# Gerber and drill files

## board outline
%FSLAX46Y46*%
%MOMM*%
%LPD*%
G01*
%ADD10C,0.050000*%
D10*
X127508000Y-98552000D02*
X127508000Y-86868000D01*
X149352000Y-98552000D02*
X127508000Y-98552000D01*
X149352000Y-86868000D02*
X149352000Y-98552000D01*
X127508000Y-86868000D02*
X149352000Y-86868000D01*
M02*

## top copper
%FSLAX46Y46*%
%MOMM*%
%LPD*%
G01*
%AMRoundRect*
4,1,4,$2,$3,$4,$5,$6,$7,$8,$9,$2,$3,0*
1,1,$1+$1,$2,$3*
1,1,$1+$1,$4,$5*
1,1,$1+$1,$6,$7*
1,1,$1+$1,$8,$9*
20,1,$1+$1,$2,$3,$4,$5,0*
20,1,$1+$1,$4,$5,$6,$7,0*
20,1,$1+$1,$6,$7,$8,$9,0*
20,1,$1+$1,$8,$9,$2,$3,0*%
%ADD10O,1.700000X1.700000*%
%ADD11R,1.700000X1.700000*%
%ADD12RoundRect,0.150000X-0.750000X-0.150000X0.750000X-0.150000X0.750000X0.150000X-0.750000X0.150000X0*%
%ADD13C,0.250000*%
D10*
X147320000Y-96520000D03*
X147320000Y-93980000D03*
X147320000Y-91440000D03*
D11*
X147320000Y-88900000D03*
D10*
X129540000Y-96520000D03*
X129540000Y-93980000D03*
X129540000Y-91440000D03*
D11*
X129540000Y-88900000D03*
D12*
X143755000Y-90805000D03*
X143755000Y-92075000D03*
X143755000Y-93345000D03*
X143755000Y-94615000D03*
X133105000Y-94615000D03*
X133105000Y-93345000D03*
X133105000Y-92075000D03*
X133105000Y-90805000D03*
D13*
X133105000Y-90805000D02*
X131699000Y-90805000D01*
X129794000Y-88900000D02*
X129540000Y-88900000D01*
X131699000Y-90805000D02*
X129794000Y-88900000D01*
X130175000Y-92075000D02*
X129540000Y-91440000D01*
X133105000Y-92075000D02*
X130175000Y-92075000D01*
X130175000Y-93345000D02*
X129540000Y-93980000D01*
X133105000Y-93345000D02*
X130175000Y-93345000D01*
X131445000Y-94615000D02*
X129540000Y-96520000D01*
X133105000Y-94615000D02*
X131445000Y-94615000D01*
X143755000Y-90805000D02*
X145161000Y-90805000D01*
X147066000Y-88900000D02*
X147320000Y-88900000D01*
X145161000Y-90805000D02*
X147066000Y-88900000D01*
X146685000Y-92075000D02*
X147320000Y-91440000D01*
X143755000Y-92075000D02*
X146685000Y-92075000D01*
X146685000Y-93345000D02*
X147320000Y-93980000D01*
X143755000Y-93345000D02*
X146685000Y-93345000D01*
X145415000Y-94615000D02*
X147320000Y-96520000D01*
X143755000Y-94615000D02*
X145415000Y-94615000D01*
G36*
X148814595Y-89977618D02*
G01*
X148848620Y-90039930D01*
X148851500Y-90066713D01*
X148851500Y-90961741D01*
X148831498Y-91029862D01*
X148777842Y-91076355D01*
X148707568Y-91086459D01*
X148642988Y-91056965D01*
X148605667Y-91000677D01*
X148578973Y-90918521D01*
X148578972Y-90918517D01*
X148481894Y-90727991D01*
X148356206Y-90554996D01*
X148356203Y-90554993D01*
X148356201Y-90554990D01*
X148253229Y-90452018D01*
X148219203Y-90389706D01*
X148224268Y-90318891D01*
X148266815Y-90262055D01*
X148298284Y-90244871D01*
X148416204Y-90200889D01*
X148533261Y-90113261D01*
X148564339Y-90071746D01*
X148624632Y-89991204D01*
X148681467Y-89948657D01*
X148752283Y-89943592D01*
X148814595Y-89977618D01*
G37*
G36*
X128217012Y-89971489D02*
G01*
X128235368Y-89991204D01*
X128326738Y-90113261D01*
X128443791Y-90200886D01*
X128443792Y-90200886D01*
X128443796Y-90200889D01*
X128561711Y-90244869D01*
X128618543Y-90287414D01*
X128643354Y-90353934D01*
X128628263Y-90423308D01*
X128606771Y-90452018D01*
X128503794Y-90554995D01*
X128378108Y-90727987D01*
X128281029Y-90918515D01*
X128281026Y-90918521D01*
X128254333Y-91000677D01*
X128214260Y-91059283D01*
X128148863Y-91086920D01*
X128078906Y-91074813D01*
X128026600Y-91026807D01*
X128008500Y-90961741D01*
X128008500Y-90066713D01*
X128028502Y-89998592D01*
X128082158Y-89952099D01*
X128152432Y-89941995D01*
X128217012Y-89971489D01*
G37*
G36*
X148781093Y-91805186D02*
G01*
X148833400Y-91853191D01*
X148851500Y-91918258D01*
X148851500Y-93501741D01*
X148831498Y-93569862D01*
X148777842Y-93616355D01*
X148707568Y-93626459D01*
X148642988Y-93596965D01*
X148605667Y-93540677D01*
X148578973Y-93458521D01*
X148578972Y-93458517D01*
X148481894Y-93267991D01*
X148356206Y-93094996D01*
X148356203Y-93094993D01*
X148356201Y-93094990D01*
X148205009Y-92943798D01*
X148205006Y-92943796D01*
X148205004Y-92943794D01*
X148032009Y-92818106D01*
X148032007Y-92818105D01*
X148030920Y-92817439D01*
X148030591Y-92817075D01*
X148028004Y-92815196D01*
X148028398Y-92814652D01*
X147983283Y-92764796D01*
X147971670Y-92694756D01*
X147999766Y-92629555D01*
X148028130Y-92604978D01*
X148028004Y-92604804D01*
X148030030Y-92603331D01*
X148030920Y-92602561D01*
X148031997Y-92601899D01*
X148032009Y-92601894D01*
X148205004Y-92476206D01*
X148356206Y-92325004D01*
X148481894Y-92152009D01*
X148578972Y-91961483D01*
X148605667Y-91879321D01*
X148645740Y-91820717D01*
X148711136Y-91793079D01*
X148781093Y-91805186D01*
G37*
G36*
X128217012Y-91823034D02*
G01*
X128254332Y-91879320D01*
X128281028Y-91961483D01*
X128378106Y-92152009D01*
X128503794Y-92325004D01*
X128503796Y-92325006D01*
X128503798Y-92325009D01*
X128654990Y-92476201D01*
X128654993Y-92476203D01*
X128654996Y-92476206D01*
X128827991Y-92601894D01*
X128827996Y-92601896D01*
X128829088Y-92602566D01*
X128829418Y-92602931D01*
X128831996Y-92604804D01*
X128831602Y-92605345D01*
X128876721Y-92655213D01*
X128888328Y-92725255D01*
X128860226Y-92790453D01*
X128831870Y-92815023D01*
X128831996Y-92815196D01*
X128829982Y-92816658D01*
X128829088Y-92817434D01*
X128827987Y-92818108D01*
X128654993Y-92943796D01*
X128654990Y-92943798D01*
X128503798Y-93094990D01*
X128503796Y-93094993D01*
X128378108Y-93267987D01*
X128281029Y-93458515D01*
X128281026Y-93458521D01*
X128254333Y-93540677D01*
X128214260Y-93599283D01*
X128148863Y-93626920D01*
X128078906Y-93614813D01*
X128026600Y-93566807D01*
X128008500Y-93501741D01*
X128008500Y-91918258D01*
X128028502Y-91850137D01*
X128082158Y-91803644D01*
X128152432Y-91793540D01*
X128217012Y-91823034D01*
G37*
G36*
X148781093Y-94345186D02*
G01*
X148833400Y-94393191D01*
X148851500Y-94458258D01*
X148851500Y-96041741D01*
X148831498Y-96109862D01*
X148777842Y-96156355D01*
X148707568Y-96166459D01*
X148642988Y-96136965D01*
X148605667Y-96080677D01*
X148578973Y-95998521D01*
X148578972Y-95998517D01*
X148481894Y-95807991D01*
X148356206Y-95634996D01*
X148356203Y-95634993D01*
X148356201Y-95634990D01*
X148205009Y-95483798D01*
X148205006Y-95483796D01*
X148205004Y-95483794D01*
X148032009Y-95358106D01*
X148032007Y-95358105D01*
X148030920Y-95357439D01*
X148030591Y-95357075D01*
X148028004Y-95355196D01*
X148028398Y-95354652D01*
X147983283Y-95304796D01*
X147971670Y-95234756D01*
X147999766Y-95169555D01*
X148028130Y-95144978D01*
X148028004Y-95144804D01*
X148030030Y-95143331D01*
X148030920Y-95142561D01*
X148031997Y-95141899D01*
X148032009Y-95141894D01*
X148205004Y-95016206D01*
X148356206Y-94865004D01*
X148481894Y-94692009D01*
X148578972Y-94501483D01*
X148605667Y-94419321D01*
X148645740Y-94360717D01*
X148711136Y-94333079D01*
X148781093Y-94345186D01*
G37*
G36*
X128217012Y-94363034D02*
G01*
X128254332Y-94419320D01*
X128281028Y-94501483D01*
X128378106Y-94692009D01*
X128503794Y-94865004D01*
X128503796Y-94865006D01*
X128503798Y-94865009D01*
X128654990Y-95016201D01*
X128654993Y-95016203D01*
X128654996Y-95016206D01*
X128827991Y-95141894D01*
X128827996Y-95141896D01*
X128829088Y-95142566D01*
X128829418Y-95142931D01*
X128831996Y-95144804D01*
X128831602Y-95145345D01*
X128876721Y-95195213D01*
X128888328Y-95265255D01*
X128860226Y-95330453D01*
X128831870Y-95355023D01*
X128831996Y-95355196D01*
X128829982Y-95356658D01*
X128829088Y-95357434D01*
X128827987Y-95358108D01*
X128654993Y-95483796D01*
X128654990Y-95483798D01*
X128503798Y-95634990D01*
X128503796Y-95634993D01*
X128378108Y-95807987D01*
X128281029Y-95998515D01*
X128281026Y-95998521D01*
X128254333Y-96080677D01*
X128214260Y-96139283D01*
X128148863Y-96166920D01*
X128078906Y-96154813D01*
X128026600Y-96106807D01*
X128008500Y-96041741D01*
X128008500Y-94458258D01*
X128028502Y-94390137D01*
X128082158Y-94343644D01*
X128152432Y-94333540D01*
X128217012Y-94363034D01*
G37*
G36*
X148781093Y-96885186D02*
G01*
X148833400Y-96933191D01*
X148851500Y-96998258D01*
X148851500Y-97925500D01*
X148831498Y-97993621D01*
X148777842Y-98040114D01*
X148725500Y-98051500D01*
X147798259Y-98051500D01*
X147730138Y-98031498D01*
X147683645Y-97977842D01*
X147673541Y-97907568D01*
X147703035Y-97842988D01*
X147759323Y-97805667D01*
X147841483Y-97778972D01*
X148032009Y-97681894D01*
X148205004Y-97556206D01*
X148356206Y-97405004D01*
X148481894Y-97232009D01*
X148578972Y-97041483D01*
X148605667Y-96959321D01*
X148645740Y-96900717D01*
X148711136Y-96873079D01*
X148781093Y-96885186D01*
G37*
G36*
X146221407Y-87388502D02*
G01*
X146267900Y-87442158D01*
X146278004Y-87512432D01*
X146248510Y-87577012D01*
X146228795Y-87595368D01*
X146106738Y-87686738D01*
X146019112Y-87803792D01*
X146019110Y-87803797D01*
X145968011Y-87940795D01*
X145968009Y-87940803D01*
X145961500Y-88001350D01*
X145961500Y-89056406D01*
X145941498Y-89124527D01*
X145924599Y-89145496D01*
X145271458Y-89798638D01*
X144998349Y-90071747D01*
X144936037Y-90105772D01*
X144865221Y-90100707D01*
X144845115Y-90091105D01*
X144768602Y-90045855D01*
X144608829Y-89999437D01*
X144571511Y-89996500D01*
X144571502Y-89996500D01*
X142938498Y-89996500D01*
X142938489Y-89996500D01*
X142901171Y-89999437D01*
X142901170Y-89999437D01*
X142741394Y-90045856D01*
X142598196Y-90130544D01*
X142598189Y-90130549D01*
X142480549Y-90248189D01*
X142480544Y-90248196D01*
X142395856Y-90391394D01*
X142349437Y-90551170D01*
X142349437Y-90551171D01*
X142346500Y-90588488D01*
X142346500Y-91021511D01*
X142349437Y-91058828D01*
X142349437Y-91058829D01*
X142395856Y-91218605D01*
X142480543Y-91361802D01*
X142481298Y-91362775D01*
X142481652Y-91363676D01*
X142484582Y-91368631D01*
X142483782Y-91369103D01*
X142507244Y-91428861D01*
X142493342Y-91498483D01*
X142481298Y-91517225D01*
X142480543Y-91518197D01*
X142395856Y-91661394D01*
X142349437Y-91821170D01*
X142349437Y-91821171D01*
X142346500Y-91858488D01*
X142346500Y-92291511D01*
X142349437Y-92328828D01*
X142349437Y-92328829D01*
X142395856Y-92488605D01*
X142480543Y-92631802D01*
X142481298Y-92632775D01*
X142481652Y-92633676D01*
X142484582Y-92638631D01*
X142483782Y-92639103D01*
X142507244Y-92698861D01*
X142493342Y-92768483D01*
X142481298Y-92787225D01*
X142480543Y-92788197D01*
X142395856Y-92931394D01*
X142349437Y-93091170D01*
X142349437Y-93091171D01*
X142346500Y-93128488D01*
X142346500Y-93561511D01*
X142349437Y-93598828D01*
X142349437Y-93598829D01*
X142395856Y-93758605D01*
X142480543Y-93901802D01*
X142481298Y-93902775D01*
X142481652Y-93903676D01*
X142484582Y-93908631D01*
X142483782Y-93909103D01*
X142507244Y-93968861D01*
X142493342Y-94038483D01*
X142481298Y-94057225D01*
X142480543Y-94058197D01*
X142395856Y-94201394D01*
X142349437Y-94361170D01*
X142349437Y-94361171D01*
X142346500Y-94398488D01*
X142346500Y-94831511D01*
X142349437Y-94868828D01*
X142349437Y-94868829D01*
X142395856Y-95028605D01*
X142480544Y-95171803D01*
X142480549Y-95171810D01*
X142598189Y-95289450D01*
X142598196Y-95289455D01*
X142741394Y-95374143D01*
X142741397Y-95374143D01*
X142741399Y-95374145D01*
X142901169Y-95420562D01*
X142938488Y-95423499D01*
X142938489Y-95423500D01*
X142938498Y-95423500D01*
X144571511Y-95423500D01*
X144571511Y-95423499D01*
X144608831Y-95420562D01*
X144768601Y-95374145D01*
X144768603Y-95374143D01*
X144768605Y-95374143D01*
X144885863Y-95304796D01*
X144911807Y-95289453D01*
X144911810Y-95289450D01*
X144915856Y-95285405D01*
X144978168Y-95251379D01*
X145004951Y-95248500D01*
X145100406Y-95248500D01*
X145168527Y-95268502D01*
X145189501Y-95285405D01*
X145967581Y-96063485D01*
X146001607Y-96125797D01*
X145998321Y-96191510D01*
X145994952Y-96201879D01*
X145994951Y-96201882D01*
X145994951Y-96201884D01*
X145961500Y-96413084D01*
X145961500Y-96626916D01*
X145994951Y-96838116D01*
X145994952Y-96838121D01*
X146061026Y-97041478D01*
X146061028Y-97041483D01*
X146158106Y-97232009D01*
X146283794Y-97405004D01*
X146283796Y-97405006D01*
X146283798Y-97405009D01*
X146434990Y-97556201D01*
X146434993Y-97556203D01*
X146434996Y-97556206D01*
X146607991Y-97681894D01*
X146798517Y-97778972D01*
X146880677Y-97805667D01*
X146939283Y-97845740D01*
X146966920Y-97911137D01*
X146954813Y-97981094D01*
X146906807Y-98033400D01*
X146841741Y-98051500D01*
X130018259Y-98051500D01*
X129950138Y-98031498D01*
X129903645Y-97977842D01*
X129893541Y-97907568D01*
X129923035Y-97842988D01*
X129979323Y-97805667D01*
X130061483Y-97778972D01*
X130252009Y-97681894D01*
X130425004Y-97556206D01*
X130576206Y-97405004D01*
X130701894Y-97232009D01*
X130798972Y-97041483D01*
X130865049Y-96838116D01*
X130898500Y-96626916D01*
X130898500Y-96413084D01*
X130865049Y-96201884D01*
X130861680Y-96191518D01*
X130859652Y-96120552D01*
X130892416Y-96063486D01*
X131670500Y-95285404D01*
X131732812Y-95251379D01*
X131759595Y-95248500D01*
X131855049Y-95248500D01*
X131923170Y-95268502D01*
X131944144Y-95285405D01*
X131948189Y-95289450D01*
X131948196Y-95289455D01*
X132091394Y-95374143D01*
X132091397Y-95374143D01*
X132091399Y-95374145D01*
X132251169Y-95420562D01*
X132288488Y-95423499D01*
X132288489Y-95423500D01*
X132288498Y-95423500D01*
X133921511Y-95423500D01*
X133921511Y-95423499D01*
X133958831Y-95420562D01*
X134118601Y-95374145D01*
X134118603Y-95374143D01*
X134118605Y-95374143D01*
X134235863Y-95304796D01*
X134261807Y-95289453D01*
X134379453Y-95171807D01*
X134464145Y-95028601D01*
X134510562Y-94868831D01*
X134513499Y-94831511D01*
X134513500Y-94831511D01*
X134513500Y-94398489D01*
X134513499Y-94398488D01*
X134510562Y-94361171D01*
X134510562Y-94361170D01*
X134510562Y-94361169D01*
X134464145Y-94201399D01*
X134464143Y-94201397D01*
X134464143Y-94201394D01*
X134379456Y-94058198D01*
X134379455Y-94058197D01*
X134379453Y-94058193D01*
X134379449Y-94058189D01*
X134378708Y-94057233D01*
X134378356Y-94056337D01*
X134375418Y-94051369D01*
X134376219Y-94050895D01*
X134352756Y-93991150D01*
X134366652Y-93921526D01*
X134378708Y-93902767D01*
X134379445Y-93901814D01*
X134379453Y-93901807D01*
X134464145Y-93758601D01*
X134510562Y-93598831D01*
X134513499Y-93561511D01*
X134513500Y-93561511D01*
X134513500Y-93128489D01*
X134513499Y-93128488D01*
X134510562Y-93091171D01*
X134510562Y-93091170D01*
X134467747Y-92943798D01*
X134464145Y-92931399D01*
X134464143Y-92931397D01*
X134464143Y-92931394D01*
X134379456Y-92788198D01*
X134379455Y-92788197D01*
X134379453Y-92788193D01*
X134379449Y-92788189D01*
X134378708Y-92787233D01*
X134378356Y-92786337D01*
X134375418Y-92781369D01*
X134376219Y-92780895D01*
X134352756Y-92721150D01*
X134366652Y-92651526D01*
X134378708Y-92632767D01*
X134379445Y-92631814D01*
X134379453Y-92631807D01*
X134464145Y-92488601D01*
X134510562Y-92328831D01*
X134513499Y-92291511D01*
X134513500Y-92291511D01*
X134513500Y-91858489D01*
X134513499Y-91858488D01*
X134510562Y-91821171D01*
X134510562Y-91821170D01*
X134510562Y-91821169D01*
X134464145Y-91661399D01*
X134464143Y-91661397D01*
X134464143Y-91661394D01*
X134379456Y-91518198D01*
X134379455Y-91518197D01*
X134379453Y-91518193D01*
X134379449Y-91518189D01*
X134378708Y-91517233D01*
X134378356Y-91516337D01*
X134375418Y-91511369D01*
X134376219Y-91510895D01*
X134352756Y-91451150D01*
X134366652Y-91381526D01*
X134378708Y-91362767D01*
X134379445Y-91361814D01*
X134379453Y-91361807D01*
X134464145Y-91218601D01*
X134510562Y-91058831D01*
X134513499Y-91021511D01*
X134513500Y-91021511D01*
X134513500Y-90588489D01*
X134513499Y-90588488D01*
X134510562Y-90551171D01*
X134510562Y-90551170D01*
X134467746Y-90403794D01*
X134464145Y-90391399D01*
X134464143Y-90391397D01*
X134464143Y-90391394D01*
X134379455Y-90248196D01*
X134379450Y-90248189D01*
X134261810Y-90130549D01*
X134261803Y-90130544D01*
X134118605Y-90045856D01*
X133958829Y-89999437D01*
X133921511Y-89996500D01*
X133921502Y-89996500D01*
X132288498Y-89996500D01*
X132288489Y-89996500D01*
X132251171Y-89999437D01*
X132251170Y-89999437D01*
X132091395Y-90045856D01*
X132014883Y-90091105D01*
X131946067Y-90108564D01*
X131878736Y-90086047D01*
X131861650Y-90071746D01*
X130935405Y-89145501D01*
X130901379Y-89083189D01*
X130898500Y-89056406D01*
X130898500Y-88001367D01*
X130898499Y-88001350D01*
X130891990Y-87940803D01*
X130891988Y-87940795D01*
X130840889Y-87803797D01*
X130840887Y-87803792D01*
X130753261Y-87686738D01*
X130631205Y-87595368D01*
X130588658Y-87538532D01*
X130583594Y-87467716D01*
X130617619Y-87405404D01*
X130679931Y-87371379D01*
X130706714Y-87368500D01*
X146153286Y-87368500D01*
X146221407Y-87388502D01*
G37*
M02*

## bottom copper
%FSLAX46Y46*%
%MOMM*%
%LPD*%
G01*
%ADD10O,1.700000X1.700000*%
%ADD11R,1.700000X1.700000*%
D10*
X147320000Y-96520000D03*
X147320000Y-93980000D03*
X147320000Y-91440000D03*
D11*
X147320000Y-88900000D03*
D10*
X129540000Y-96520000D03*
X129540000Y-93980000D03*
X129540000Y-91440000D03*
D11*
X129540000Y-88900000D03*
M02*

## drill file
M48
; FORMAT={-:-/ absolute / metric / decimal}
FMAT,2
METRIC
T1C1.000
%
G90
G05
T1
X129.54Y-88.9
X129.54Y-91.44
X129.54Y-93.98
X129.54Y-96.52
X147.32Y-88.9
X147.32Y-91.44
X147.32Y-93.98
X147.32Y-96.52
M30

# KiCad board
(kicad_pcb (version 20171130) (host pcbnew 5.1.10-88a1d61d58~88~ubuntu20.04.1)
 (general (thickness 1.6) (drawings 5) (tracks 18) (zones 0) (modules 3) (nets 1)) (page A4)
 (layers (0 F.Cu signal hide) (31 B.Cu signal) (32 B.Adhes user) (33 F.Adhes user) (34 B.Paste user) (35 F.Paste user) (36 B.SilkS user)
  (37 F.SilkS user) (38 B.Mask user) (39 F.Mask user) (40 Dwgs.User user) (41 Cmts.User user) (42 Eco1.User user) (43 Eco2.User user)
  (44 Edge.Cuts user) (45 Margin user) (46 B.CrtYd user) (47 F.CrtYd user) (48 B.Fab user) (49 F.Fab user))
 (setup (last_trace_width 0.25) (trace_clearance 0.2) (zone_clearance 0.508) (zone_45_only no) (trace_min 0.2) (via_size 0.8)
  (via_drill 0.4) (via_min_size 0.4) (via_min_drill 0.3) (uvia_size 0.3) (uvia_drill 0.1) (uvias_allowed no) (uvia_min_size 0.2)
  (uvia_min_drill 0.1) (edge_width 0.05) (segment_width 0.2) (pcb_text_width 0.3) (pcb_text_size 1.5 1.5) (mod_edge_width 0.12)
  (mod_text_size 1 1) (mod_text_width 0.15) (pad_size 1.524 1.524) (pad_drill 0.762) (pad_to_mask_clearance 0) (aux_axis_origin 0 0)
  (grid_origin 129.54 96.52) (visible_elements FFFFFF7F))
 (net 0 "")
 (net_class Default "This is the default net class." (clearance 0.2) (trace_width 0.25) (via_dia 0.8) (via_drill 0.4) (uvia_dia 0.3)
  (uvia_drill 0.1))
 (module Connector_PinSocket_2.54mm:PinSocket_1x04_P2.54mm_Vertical (layer F.Cu) (at 147.32 88.9)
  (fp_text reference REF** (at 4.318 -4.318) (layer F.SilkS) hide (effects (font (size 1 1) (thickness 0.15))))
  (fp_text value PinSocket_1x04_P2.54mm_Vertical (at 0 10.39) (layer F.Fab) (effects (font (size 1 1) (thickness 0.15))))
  (pad 4 thru_hole oval (at 0 7.62) (size 1.7 1.7) (drill 1) (layers *.Cu *.Mask))
  (pad 3 thru_hole oval (at 0 5.08) (size 1.7 1.7) (drill 1) (layers *.Cu *.Mask))
  (pad 2 thru_hole oval (at 0 2.54) (size 1.7 1.7) (drill 1) (layers *.Cu *.Mask))
  (pad 1 thru_hole rect (at 0 0) (size 1.7 1.7) (drill 1) (layers *.Cu *.Mask)))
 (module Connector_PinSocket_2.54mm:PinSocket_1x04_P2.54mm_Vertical (layer F.Cu) (at 129.54 88.9)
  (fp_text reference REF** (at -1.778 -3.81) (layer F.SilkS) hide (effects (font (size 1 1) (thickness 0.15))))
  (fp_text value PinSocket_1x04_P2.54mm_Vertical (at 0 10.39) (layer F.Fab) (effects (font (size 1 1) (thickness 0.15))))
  (pad 4 thru_hole oval (at 0 7.62) (size 1.7 1.7) (drill 1) (layers *.Cu *.Mask))
  (pad 3 thru_hole oval (at 0 5.08) (size 1.7 1.7) (drill 1) (layers *.Cu *.Mask))
  (pad 2 thru_hole oval (at 0 2.54) (size 1.7 1.7) (drill 1) (layers *.Cu *.Mask))
  (pad 1 thru_hole rect (at 0 0) (size 1.7 1.7) (drill 1) (layers *.Cu *.Mask)))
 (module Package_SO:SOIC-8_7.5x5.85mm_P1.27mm (layer F.Cu) (at 138.43 92.71)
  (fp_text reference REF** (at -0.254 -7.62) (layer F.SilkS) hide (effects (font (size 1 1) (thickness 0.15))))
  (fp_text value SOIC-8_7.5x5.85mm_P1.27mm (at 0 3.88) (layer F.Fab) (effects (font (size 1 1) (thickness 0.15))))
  (pad 8 smd roundrect (at 5.325 -1.905) (size 1.8 0.6) (layers F.Cu F.Paste F.Mask) (roundrect_rratio 0.25))
  (pad 7 smd roundrect (at 5.325 -0.635) (size 1.8 0.6) (layers F.Cu F.Paste F.Mask) (roundrect_rratio 0.25))
  (pad 6 smd roundrect (at 5.325 0.635) (size 1.8 0.6) (layers F.Cu F.Paste F.Mask) (roundrect_rratio 0.25))
  (pad 5 smd roundrect (at 5.325 1.905) (size 1.8 0.6) (layers F.Cu F.Paste F.Mask) (roundrect_rratio 0.25))
  (pad 4 smd roundrect (at -5.325 1.905) (size 1.8 0.6) (layers F.Cu F.Paste F.Mask) (roundrect_rratio 0.25))
  (pad 3 smd roundrect (at -5.325 0.635) (size 1.8 0.6) (layers F.Cu F.Paste F.Mask) (roundrect_rratio 0.25))
  (pad 2 smd roundrect (at -5.325 -0.635) (size 1.8 0.6) (layers F.Cu F.Paste F.Mask) (roundrect_rratio 0.25))
  (pad 1 smd roundrect (at -5.325 -1.905) (size 1.8 0.6) (layers F.Cu F.Paste F.Mask) (roundrect_rratio 0.25)))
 (gr_line (start 127.508 98.552) (end 127.508 86.868) (layer Edge.Cuts) (width 0.05))
 (gr_line (start 149.352 98.552) (end 127.508 98.552) (layer Edge.Cuts) (width 0.05))
 (gr_line (start 149.352 86.868) (end 149.352 98.552) (layer Edge.Cuts) (width 0.05))
 (gr_line (start 127.508 86.868) (end 149.352 86.868) (layer Edge.Cuts) (width 0.05))
 (segment (start 133.105 90.805) (end 131.699 90.805) (width 0.25) (layer F.Cu) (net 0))
 (segment (start 129.794 88.9) (end 129.54 88.9) (width 0.25) (layer F.Cu) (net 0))
 (segment (start 131.699 90.805) (end 129.794 88.9) (width 0.25) (layer F.Cu) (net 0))
 (segment (start 130.175 92.075) (end 129.54 91.44) (width 0.25) (layer F.Cu) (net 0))
 (segment (start 133.105 92.075) (end 130.175 92.075) (width 0.25) (layer F.Cu) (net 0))
 (segment (start 130.175 93.345) (end 129.54 93.98) (width 0.25) (layer F.Cu) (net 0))
 (segment (start 133.105 93.345) (end 130.175 93.345) (width 0.25) (layer F.Cu) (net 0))
 (segment (start 131.445 94.615) (end 129.54 96.52) (width 0.25) (layer F.Cu) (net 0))
 (segment (start 133.105 94.615) (end 131.445 94.615) (width 0.25) (layer F.Cu) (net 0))
 (segment (start 143.755 90.805) (end 145.161 90.805) (width 0.25) (layer F.Cu) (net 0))
 (segment (start 147.066 88.9) (end 147.32 88.9) (width 0.25) (layer F.Cu) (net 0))
 (segment (start 145.161 90.805) (end 147.066 88.9) (width 0.25) (layer F.Cu) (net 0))
 (segment (start 146.685 92.075) (end 147.32 91.44) (width 0.25) (layer F.Cu) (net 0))
 (segment (start 143.755 92.075) (end 146.685 92.075) (width 0.25) (layer F.Cu) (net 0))
 (segment (start 146.685 93.345) (end 147.32 93.98) (width 0.25) (layer F.Cu) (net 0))
 (segment (start 143.755 93.345) (end 146.685 93.345) (width 0.25) (layer F.Cu) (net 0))
 (segment (start 145.415 94.615) (end 147.32 96.52) (width 0.25) (layer F.Cu) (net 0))
 (segment (start 143.755 94.615) (end 145.415 94.615) (width 0.25) (layer F.Cu) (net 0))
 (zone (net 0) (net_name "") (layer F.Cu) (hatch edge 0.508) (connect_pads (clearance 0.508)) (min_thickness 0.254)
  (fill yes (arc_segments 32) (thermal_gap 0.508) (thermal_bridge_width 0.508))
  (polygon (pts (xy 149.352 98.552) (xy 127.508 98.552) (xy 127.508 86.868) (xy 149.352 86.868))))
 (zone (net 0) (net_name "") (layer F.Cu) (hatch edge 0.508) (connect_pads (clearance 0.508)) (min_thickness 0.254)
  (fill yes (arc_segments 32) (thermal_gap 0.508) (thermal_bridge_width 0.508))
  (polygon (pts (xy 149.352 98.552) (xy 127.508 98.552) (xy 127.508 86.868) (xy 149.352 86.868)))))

